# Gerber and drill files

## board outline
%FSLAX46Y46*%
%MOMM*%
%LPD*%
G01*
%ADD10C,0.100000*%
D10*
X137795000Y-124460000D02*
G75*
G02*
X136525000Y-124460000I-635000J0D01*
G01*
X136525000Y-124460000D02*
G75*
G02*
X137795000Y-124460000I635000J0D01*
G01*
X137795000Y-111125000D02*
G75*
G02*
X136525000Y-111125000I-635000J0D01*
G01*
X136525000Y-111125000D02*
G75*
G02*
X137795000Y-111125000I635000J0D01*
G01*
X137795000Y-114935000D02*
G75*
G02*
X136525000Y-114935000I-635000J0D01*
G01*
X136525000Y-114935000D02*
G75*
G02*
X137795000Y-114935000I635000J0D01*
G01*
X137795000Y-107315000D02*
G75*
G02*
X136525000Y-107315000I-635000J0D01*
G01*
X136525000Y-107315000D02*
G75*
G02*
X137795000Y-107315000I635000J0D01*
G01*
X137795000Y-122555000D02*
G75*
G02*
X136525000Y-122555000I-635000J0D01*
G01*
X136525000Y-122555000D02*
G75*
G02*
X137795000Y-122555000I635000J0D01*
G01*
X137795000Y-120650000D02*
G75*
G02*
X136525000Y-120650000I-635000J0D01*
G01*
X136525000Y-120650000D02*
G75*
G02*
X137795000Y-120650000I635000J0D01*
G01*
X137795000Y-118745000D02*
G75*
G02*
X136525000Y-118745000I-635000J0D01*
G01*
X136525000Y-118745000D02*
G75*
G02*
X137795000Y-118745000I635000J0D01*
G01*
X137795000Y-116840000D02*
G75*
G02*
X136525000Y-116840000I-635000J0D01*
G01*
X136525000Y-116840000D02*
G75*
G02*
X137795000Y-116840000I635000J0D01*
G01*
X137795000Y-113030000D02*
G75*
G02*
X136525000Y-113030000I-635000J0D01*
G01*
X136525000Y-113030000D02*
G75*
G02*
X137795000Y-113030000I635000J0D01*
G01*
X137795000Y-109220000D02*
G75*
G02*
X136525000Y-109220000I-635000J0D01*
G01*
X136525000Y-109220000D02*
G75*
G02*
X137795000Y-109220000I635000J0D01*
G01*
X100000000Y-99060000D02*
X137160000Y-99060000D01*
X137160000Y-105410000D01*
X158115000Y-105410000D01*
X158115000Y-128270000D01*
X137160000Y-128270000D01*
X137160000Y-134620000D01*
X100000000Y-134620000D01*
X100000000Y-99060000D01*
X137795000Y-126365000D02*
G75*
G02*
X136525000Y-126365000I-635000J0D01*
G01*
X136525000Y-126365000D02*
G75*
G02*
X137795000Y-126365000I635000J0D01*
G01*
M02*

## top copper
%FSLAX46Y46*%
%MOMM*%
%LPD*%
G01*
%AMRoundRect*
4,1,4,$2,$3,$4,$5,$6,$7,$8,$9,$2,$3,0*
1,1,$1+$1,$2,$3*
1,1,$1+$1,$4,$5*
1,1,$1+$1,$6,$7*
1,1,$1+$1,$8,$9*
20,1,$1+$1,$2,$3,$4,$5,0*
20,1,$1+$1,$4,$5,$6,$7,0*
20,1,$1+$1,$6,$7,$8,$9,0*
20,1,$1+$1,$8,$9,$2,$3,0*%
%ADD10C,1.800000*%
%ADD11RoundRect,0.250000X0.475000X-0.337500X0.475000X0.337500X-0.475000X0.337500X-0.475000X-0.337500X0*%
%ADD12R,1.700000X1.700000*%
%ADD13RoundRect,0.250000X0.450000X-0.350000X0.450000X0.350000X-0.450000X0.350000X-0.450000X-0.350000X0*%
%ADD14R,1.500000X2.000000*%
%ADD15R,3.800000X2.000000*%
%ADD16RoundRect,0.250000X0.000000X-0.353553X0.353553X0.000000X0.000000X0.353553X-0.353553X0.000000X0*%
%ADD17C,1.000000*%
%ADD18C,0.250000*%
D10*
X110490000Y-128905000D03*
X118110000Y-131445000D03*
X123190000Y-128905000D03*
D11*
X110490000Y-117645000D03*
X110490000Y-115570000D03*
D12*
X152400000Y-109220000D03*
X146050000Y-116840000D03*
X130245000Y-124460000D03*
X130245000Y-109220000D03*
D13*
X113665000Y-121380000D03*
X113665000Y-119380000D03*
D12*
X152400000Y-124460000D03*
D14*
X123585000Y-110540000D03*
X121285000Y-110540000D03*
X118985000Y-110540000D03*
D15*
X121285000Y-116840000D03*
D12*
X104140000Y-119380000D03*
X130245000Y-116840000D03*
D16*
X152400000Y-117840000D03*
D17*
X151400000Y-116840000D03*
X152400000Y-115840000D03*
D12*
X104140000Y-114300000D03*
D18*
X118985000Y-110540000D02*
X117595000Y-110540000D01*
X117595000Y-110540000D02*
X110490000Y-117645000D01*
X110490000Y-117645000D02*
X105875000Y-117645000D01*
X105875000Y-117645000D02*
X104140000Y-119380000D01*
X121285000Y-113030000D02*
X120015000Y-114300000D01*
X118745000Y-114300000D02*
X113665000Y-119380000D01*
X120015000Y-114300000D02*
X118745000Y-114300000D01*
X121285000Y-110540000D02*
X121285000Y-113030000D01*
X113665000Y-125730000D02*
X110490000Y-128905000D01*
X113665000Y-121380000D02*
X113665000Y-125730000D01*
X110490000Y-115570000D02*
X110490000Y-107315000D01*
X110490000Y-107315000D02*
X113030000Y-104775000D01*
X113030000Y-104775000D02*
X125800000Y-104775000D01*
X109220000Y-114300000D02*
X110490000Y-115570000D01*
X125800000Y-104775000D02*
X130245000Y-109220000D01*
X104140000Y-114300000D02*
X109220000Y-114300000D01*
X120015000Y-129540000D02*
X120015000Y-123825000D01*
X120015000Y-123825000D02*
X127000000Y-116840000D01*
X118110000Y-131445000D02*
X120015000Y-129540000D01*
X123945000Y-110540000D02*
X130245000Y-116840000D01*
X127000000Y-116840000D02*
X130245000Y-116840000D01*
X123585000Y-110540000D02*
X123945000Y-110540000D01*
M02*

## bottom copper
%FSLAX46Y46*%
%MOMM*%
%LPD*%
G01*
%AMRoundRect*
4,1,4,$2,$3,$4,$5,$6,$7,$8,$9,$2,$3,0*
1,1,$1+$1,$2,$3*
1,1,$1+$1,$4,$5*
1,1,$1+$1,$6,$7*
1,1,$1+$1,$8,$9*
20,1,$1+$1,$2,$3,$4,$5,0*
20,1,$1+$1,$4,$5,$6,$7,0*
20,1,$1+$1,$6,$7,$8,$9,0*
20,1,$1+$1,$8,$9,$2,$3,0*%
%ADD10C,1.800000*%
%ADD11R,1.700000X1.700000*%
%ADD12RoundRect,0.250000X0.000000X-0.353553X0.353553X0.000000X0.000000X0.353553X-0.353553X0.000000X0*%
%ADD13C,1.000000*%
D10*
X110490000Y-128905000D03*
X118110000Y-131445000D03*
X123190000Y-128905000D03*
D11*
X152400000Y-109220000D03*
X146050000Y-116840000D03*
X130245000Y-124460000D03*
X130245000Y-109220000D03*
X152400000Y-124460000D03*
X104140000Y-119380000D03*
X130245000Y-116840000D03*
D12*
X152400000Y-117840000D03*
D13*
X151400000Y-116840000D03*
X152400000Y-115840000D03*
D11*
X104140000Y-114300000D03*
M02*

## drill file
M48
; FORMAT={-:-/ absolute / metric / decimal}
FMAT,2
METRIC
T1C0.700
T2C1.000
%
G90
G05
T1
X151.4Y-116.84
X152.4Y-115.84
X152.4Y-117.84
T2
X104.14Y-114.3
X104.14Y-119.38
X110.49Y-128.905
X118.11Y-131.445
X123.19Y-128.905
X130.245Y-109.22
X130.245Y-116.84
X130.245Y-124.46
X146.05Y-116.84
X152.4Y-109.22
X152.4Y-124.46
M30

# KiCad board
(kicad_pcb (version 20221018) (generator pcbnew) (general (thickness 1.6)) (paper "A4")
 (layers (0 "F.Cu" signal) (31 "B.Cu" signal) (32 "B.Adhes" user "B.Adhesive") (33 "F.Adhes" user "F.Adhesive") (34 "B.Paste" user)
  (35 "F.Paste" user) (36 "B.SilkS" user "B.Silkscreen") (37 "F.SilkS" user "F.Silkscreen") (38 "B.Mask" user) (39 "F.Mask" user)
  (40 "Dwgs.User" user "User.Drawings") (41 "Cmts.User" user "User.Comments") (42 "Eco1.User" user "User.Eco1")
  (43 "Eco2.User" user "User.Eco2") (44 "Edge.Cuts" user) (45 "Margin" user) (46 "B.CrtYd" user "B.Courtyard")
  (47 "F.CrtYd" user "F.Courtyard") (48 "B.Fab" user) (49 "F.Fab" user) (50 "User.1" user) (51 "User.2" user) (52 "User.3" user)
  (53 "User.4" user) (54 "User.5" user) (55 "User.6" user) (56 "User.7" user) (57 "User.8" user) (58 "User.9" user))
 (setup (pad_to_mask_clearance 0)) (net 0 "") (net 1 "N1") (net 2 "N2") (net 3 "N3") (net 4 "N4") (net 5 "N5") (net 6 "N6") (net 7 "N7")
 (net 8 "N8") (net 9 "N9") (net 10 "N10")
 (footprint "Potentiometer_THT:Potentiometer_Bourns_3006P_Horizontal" (layer "F.Cu") (at 110.49 128.905 180)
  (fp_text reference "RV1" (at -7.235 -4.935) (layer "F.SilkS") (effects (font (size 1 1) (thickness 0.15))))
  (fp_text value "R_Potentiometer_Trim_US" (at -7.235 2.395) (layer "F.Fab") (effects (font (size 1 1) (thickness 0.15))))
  (pad "1" thru_hole circle (at 0 0 180) (size 1.8 1.8) (drill 1) (layers "*.Cu" "*.Mask") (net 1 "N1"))
  (pad "2" thru_hole circle (at -7.62 -2.54 180) (size 1.8 1.8) (drill 1) (layers "*.Cu" "*.Mask") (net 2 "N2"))
  (pad "3" thru_hole circle (at -12.7 0 180) (size 1.8 1.8) (drill 1) (layers "*.Cu" "*.Mask") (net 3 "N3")))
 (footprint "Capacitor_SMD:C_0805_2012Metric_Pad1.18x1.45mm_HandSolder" (layer "F.Cu") (at 110.49 116.6075 90)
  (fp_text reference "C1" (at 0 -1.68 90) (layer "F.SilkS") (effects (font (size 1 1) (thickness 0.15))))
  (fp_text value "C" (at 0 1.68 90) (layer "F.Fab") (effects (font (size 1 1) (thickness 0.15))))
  (pad "1" smd roundrect (at -1.0375 0 90) (size 1.175 1.45) (layers "F.Cu" "F.Paste" "F.Mask") (roundrect_rratio 0.212766) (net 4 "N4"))
  (pad "2" smd roundrect (at 1.0375 0 90) (size 1.175 1.45) (layers "F.Cu" "F.Paste" "F.Mask") (roundrect_rratio 0.212766) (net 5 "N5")))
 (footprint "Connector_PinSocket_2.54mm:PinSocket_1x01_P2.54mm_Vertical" (layer "F.Cu") (at 152.4 109.22)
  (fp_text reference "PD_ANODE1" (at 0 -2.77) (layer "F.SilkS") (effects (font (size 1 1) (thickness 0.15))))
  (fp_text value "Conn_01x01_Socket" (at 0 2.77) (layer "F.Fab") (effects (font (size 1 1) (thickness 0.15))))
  (pad "1" thru_hole rect (at 0 0) (size 1.7 1.7) (drill 1) (layers "*.Cu" "*.Mask") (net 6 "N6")))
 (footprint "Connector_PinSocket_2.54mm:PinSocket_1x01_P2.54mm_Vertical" (layer "F.Cu") (at 146.05 116.84)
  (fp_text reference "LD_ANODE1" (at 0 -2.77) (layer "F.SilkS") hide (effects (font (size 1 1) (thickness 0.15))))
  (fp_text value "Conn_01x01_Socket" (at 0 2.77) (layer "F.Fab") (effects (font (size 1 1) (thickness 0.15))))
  (pad "1" thru_hole rect (at 0 0) (size 1.7 1.7) (drill 1) (layers "*.Cu" "*.Mask") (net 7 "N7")))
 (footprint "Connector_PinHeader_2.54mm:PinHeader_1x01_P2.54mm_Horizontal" (layer "F.Cu") (at 130.245 124.46)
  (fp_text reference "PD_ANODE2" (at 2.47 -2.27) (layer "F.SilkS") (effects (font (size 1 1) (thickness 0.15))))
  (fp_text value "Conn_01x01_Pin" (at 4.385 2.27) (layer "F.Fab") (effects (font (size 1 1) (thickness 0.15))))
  (pad "1" thru_hole rect (at 0 0) (size 1.7 1.7) (drill 1) (layers "*.Cu" "*.Mask") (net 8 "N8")))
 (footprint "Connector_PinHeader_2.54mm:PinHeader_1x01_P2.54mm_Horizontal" (layer "F.Cu") (at 130.245 109.22)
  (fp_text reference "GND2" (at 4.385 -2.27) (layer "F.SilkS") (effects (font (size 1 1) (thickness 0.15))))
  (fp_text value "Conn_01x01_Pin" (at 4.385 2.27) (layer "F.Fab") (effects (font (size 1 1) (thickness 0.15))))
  (pad "1" thru_hole rect (at 0 0) (size 1.7 1.7) (drill 1) (layers "*.Cu" "*.Mask") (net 5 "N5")))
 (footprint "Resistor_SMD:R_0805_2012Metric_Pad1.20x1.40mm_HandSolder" (layer "F.Cu") (at 113.665 120.38 90)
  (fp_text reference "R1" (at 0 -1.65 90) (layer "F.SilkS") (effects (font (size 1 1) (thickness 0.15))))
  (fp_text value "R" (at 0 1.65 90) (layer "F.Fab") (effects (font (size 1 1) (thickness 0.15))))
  (pad "1" smd roundrect (at -1 0 90) (size 1.2 1.4) (layers "F.Cu" "F.Paste" "F.Mask") (roundrect_rratio 0.208333) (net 1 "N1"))
  (pad "2" smd roundrect (at 1 0 90) (size 1.2 1.4) (layers "F.Cu" "F.Paste" "F.Mask") (roundrect_rratio 0.208333) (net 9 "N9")))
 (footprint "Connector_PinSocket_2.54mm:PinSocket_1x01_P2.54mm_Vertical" (layer "F.Cu") (at 152.4 124.46)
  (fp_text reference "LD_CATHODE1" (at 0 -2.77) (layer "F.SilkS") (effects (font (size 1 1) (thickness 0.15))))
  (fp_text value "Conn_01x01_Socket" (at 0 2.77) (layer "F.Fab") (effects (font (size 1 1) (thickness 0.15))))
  (pad "1" thru_hole rect (at 0 0) (size 1.7 1.7) (drill 1) (layers "*.Cu" "*.Mask") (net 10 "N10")))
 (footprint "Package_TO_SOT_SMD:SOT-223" (layer "F.Cu") (at 121.285 113.69 -90)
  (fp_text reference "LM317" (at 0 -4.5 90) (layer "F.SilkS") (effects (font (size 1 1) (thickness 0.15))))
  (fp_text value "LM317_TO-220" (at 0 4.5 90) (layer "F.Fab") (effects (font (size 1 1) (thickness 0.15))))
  (pad "1" smd rect (at -3.15 -2.3 270) (size 2 1.5) (layers "F.Cu" "F.Paste" "F.Mask") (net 2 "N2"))
  (pad "2" smd rect (at -3.15 0 270) (size 2 1.5) (layers "F.Cu" "F.Paste" "F.Mask") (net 9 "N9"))
  (pad "3" smd rect (at -3.15 2.3 270) (size 2 1.5) (layers "F.Cu" "F.Paste" "F.Mask") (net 4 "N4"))
  (pad "4" smd rect (at 3.15 0 270) (size 2 3.8) (layers "F.Cu" "F.Paste" "F.Mask")))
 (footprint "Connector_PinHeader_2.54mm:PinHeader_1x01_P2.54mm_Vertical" (layer "B.Cu") (at 104.14 119.38 180)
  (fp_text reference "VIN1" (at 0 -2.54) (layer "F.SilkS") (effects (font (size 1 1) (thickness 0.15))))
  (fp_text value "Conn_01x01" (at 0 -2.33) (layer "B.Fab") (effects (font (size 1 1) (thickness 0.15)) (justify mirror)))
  (pad "1" thru_hole rect (at 0 0 180) (size 1.7 1.7) (drill 1) (layers "*.Cu" "*.Mask") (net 4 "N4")))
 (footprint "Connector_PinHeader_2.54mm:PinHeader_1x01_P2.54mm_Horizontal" (layer "B.Cu") (at 130.245 116.84)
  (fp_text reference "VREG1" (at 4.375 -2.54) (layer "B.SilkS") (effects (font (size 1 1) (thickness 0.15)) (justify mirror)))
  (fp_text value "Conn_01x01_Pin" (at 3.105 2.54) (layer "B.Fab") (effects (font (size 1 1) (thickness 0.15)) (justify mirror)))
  (pad "1" thru_hole rect (at 0 0) (size 1.7 1.7) (drill 1) (layers "*.Cu" "*.Mask") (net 2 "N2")))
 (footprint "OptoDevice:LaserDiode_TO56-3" (layer "B.Cu") (at 152.4 117.84 90)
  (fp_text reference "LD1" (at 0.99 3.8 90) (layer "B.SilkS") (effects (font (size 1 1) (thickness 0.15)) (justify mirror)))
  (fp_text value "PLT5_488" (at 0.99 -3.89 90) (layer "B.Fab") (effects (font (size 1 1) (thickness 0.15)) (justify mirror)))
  (pad "1" thru_hole roundrect (at 0 0 45) (size 1 1) (drill 0.7) (layers "*.Cu" "*.Mask") (roundrect_rratio 0.25) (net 10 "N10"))
  (pad "2" thru_hole circle (at 1 -1 90) (size 1 1) (drill 0.7) (layers "*.Cu" "*.Mask") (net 7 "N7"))
  (pad "3" thru_hole circle (at 2 0 90) (size 1 1) (drill 0.7) (layers "*.Cu" "*.Mask") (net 6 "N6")))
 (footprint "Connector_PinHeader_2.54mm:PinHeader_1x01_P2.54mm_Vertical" (layer "B.Cu") (at 104.14 114.3 180)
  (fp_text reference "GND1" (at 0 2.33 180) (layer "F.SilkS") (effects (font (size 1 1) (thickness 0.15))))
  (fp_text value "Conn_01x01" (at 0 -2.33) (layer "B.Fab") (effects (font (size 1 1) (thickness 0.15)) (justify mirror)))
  (pad "1" thru_hole rect (at 0 0 180) (size 1.7 1.7) (drill 1) (layers "*.Cu" "*.Mask") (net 5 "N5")))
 (gr_circle (center 137.16 124.46) (end 137.795 124.46) (stroke (width 0.1) (type default)) (fill none) (layer "Edge.Cuts"))
 (gr_circle (center 137.16 111.125) (end 137.795 111.125) (stroke (width 0.1) (type default)) (fill none) (layer "Edge.Cuts"))
 (gr_circle (center 137.16 114.935) (end 137.795 114.935) (stroke (width 0.1) (type default)) (fill none) (layer "Edge.Cuts"))
 (gr_circle (center 137.16 107.315) (end 137.795 107.315) (stroke (width 0.1) (type default)) (fill none) (layer "Edge.Cuts"))
 (gr_circle (center 137.16 122.555) (end 137.795 122.555) (stroke (width 0.1) (type default)) (fill none) (layer "Edge.Cuts"))
 (gr_circle (center 137.16 120.65) (end 137.795 120.65) (stroke (width 0.1) (type default)) (fill none) (layer "Edge.Cuts"))
 (gr_circle (center 137.16 118.745) (end 137.795 118.745) (stroke (width 0.1) (type default)) (fill none) (layer "Edge.Cuts"))
 (gr_circle (center 137.16 116.84) (end 137.795 116.84) (stroke (width 0.1) (type default)) (fill none) (layer "Edge.Cuts"))
 (gr_circle (center 137.16 113.03) (end 137.795 113.03) (stroke (width 0.1) (type default)) (fill none) (layer "Edge.Cuts"))
 (gr_circle (center 137.16 109.22) (end 137.795 109.22) (stroke (width 0.1) (type default)) (fill none) (layer "Edge.Cuts"))
 (gr_poly
  (pts (xy 100 99.06) (xy 137.16 99.06) (xy 137.16 105.41) (xy 158.115 105.41) (xy 158.115 128.27) (xy 137.16 128.27) (xy 137.16 134.62)
   (xy 100 134.62))
  (stroke (width 0.1) (type solid)) (fill none) (layer "Edge.Cuts"))
 (gr_circle (center 137.16 126.365) (end 137.795 126.365) (stroke (width 0.1) (type default)) (fill none) (layer "Edge.Cuts"))
 (segment (start 118.985 110.54) (end 117.595 110.54) (width 0.25) (layer "F.Cu") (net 4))
 (segment (start 117.595 110.54) (end 110.49 117.645) (width 0.25) (layer "F.Cu") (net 4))
 (segment (start 110.49 117.645) (end 105.875 117.645) (width 0.25) (layer "F.Cu") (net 4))
 (segment (start 105.875 117.645) (end 104.14 119.38) (width 0.25) (layer "F.Cu") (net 4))
 (segment (start 121.285 113.03) (end 120.015 114.3) (width 0.25) (layer "F.Cu") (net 9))
 (segment (start 118.745 114.3) (end 113.665 119.38) (width 0.25) (layer "F.Cu") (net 9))
 (segment (start 120.015 114.3) (end 118.745 114.3) (width 0.25) (layer "F.Cu") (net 9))
 (segment (start 121.285 110.54) (end 121.285 113.03) (width 0.25) (layer "F.Cu") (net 9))
 (segment (start 113.665 125.73) (end 110.49 128.905) (width 0.25) (layer "F.Cu") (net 1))
 (segment (start 113.665 121.38) (end 113.665 125.73) (width 0.25) (layer "F.Cu") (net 1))
 (segment (start 110.49 115.57) (end 110.49 107.315) (width 0.25) (layer "F.Cu") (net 5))
 (segment (start 110.49 107.315) (end 113.03 104.775) (width 0.25) (layer "F.Cu") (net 5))
 (segment (start 113.03 104.775) (end 125.8 104.775) (width 0.25) (layer "F.Cu") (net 5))
 (segment (start 109.22 114.3) (end 110.49 115.57) (width 0.25) (layer "F.Cu") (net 5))
 (segment (start 125.8 104.775) (end 130.245 109.22) (width 0.25) (layer "F.Cu") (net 5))
 (segment (start 104.14 114.3) (end 109.22 114.3) (width 0.25) (layer "F.Cu") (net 5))
 (segment (start 120.015 129.54) (end 120.015 123.825) (width 0.25) (layer "F.Cu") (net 2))
 (segment (start 120.015 123.825) (end 127 116.84) (width 0.25) (layer "F.Cu") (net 2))
 (segment (start 118.11 131.445) (end 120.015 129.54) (width 0.25) (layer "F.Cu") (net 2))
 (segment (start 123.945 110.54) (end 130.245 116.84) (width 0.25) (layer "F.Cu") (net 2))
 (segment (start 127 116.84) (end 130.245 116.84) (width 0.25) (layer "F.Cu") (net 2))
 (segment (start 123.585 110.54) (end 123.945 110.54) (width 0.25) (layer "F.Cu") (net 2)))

